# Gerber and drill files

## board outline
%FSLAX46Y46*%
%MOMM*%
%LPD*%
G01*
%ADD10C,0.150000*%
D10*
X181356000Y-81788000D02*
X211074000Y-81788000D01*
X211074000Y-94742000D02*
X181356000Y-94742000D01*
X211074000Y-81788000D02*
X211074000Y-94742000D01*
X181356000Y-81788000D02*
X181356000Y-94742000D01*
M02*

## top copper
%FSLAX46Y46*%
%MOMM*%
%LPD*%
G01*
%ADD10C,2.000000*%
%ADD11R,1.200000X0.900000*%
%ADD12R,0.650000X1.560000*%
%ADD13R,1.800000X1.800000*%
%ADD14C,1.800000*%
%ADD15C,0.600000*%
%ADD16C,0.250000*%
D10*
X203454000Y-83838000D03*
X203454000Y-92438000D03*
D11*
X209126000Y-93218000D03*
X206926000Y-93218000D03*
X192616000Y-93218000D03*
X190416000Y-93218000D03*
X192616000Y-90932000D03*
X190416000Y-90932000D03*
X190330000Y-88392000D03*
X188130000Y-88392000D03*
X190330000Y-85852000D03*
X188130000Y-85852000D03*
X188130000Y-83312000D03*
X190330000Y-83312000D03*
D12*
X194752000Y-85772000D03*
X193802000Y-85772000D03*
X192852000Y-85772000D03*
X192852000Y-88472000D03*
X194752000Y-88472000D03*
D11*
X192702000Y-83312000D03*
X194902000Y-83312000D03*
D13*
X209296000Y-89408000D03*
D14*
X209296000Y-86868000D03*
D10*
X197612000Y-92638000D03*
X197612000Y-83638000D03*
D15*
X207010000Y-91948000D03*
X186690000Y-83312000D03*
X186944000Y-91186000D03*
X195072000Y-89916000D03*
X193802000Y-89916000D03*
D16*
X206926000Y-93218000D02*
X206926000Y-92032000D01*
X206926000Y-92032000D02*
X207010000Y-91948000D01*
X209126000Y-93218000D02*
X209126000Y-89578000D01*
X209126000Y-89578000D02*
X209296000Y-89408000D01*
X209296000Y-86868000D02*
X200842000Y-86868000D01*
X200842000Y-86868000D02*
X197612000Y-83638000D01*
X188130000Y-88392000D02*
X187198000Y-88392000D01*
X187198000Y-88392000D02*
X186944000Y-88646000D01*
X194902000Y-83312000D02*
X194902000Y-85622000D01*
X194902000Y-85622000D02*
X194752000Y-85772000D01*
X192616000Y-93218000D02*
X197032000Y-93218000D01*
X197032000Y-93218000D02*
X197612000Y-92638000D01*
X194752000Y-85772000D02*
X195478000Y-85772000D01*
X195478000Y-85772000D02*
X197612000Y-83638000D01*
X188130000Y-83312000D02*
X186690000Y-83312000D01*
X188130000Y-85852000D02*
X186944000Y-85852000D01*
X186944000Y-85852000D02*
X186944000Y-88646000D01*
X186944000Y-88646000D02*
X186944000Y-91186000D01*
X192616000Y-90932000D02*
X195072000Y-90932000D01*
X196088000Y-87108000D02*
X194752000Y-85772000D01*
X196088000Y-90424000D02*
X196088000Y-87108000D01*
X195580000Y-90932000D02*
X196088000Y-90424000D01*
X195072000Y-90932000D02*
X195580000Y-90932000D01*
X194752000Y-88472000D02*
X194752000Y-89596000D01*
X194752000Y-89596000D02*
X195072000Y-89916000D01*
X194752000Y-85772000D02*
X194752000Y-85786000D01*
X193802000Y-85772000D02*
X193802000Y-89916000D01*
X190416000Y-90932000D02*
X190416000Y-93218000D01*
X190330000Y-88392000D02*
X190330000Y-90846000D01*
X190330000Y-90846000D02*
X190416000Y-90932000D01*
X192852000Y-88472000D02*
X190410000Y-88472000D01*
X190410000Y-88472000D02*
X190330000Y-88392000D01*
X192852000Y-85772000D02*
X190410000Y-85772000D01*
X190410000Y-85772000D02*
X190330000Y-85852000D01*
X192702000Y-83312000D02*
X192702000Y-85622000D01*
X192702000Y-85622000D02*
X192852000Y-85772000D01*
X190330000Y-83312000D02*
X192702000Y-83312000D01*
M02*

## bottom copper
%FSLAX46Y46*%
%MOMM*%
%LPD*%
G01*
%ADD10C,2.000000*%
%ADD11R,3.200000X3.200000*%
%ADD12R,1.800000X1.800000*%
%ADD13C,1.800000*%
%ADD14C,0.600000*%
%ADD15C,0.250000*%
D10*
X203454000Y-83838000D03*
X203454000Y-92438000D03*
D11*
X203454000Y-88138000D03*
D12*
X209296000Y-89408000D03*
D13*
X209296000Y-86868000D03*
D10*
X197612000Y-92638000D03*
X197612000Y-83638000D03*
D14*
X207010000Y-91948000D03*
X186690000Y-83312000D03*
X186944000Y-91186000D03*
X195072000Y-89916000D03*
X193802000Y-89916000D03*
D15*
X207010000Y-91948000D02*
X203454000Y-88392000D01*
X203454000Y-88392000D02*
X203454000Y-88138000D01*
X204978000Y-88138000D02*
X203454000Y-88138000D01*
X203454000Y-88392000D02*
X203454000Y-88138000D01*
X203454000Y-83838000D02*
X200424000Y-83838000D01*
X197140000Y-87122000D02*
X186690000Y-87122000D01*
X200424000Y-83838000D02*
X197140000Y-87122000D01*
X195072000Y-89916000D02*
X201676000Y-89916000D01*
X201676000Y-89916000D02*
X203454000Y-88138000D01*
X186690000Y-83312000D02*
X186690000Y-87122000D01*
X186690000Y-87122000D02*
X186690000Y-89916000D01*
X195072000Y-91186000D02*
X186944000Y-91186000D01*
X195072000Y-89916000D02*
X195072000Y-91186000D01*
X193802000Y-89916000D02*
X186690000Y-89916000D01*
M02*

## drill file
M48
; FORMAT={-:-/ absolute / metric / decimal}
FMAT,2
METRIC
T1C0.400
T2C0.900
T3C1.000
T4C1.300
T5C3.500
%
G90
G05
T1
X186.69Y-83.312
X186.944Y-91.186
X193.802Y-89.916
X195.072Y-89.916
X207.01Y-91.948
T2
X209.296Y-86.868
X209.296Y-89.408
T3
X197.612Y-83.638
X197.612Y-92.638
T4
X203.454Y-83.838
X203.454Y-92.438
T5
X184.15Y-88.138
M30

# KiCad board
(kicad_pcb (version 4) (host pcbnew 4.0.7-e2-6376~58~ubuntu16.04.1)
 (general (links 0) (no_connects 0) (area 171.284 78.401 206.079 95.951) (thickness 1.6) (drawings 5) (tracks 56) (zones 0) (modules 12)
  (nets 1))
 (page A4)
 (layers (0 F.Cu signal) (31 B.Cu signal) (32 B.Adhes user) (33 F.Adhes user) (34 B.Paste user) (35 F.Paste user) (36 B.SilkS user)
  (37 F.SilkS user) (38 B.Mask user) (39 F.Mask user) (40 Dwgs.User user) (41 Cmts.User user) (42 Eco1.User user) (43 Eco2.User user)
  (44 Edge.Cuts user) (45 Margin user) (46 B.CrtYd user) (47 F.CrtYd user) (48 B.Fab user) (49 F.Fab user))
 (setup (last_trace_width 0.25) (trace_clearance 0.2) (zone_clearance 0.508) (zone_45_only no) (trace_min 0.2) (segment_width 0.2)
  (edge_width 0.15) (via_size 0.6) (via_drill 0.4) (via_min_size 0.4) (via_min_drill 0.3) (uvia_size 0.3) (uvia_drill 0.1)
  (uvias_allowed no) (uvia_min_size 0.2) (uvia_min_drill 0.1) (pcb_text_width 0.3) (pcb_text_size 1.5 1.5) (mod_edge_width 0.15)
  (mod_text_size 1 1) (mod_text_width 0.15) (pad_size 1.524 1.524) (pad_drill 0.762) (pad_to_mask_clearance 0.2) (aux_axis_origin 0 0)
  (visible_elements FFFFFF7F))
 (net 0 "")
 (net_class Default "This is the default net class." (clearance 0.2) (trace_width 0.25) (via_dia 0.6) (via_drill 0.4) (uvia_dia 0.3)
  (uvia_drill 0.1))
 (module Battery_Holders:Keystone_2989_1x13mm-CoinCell (layer B.Cu) (at 203.454 88.138 270)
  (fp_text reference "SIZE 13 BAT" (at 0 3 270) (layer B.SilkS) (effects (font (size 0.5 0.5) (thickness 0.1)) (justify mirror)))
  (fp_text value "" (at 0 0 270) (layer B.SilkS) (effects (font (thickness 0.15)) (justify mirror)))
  (pad 1 thru_hole circle (at -4.3 0 270) (size 2 2) (drill 1.3) (layers *.Cu *.Mask))
  (pad 1 thru_hole circle (at 4.3 0 270) (size 2 2) (drill 1.3) (layers *.Cu *.Mask))
  (pad 2 smd rect (at 0 0 270) (size 3.2 3.2) (layers B.Cu B.Mask)))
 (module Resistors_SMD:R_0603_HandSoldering (layer F.Cu) (at 208.026 93.218 180)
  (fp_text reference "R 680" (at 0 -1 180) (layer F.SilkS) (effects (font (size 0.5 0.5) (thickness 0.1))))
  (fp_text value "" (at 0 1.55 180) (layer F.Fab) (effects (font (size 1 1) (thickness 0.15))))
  (pad 1 smd rect (at -1.1 0 180) (size 1.2 0.9) (layers F.Cu F.Paste F.Mask))
  (pad 2 smd rect (at 1.1 0 180) (size 1.2 0.9) (layers F.Cu F.Paste F.Mask)))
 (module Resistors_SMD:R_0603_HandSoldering (layer F.Cu) (at 191.516 93.218 180)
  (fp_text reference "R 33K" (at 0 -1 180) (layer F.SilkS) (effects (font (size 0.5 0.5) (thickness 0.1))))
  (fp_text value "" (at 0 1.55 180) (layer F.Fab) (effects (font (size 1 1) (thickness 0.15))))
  (pad 1 smd rect (at -1.1 0 180) (size 1.2 0.9) (layers F.Cu F.Paste F.Mask))
  (pad 2 smd rect (at 1.1 0 180) (size 1.2 0.9) (layers F.Cu F.Paste F.Mask)))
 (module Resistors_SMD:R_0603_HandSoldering (layer F.Cu) (at 191.516 90.932 180)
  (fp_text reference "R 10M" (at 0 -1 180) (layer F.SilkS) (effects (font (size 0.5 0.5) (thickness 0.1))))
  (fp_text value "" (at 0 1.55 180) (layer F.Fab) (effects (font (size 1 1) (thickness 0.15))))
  (pad 1 smd rect (at -1.1 0 180) (size 1.2 0.9) (layers F.Cu F.Paste F.Mask))
  (pad 2 smd rect (at 1.1 0 180) (size 1.2 0.9) (layers F.Cu F.Paste F.Mask)))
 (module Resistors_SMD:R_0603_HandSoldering (layer F.Cu) (at 189.23 88.392 180)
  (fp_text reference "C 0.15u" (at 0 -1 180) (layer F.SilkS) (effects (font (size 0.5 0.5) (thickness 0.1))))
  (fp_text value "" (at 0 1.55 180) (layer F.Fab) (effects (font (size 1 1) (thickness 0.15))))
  (pad 1 smd rect (at -1.1 0 180) (size 1.2 0.9) (layers F.Cu F.Paste F.Mask))
  (pad 2 smd rect (at 1.1 0 180) (size 1.2 0.9) (layers F.Cu F.Paste F.Mask)))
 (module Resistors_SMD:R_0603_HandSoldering (layer F.Cu) (at 189.23 85.852 180)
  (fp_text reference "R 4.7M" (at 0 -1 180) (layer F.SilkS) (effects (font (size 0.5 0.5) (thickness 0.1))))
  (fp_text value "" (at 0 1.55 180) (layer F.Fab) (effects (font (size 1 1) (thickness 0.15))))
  (pad 1 smd rect (at -1.1 0 180) (size 1.2 0.9) (layers F.Cu F.Paste F.Mask))
  (pad 2 smd rect (at 1.1 0 180) (size 1.2 0.9) (layers F.Cu F.Paste F.Mask)))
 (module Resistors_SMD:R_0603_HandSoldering (layer F.Cu) (at 189.23 83.312)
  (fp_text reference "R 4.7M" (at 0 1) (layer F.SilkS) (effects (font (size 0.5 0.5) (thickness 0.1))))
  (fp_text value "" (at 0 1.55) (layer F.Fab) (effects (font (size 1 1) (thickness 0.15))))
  (pad 1 smd rect (at -1.1 0) (size 1.2 0.9) (layers F.Cu F.Paste F.Mask))
  (pad 2 smd rect (at 1.1 0) (size 1.2 0.9) (layers F.Cu F.Paste F.Mask)))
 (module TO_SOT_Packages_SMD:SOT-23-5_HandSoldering (layer F.Cu) (at 193.802 87.122 270)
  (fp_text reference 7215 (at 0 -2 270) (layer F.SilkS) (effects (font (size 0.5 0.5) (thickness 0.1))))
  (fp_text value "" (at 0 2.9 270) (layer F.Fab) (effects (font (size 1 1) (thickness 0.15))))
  (pad 1 smd rect (at -1.35 -0.95 270) (size 1.56 0.65) (layers F.Cu F.Paste F.Mask))
  (pad 2 smd rect (at -1.35 0 270) (size 1.56 0.65) (layers F.Cu F.Paste F.Mask))
  (pad 3 smd rect (at -1.35 0.95 270) (size 1.56 0.65) (layers F.Cu F.Paste F.Mask))
  (pad 4 smd rect (at 1.35 0.95 270) (size 1.56 0.65) (layers F.Cu F.Paste F.Mask))
  (pad 5 smd rect (at 1.35 -0.95 270) (size 1.56 0.65) (layers F.Cu F.Paste F.Mask)))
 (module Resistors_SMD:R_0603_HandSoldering (layer F.Cu) (at 193.802 83.312)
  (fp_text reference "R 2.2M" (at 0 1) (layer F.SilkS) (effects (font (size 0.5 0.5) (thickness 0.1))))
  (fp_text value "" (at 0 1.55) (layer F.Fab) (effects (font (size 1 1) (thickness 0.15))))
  (pad 1 smd rect (at -1.1 0) (size 1.2 0.9) (layers F.Cu F.Paste F.Mask))
  (pad 2 smd rect (at 1.1 0) (size 1.2 0.9) (layers F.Cu F.Paste F.Mask)))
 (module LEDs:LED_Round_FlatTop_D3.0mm (layer F.Cu) (at 209.296 89.408 90)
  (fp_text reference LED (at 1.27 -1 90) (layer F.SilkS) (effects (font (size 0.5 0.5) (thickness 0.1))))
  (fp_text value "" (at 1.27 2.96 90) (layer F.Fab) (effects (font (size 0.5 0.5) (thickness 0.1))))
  (pad 1 thru_hole rect (at 0 0 90) (size 1.8 1.8) (drill 0.9) (layers *.Cu *.Mask))
  (pad 2 thru_hole circle (at 2.54 0 90) (size 1.8 1.8) (drill 0.9) (layers *.Cu *.Mask)))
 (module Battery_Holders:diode (layer F.Cu) (at 197.612 88.138 90)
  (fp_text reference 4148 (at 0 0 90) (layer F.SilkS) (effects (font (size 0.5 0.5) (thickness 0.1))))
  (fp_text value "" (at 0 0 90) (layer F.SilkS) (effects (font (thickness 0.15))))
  (pad 1 thru_hole circle (at -4.5 0 90) (size 2 2) (drill 1) (layers *.Cu *.Mask))
  (pad 2 thru_hole circle (at 4.5 0 90) (size 2 2) (drill 1) (layers *.Cu *.Mask)))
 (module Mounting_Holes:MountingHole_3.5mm (layer F.Cu) (at 184.15 88.138)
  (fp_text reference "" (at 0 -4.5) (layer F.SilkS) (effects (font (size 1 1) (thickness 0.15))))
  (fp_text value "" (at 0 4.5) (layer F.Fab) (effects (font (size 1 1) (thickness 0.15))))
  (pad 1 np_thru_hole circle (at 0 0) (size 3.5 3.5) (drill 3.5) (layers *.Cu *.Mask)))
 (gr_line (start 181.356 81.788) (end 211.074 81.788) (angle 90) (layer Edge.Cuts) (width 0.15))
 (gr_line (start 211.074 94.742) (end 181.356 94.742) (angle 90) (layer Edge.Cuts) (width 0.15))
 (gr_line (start 211.074 81.788) (end 211.074 94.742) (angle 90) (layer Edge.Cuts) (width 0.15))
 (gr_line (start 181.356 81.788) (end 181.356 94.742) (angle 90) (layer Edge.Cuts) (width 0.15))
 (segment (start 206.926 93.218) (end 206.926 92.032) (width 0.25) (layer F.Cu) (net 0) (status 400000))
 (segment (start 207.01 91.948) (end 203.454 88.392) (width 0.25) (layer B.Cu) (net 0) (status 800000))
 (via (at 207.01 91.948) (size 0.6) (drill 0.4) (layers F.Cu B.Cu) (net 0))
 (segment (start 206.926 92.032) (end 207.01 91.948) (width 0.25) (layer F.Cu) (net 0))
 (segment (start 203.454 88.392) (end 203.454 88.138) (width 0.25) (layer B.Cu) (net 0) (status C00000))
 (segment (start 209.126 93.218) (end 209.126 89.578) (width 0.25) (layer F.Cu) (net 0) (status C00000))
 (segment (start 209.126 89.578) (end 209.296 89.408) (width 0.25) (layer F.Cu) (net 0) (status C00000))
 (segment (start 209.296 86.868) (end 200.842 86.868) (width 0.25) (layer F.Cu) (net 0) (status 400000))
 (segment (start 200.842 86.868) (end 197.612 83.638) (width 0.25) (layer F.Cu) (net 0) (status 800000))
 (segment (start 204.978 88.138) (end 203.454 88.138) (width 0.25) (layer B.Cu) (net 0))
 (segment (start 188.13 88.392) (end 187.198 88.392) (width 0.25) (layer F.Cu) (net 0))
 (segment (start 187.198 88.392) (end 186.944 88.646) (width 0.25) (layer F.Cu) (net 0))
 (segment (start 203.454 88.392) (end 203.454 88.138) (width 0.25) (layer B.Cu) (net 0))
 (segment (start 194.902 83.312) (end 194.902 85.622) (width 0.25) (layer F.Cu) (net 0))
 (segment (start 194.902 85.622) (end 194.752 85.772) (width 0.25) (layer F.Cu) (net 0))
 (segment (start 203.454 83.838) (end 200.424 83.838) (width 0.25) (layer B.Cu) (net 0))
 (segment (start 197.14 87.122) (end 186.69 87.122) (width 0.25) (layer B.Cu) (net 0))
 (segment (start 200.424 83.838) (end 197.14 87.122) (width 0.25) (layer B.Cu) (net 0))
 (segment (start 195.072 89.916) (end 201.676 89.916) (width 0.25) (layer B.Cu) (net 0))
 (segment (start 201.676 89.916) (end 203.454 88.138) (width 0.25) (layer B.Cu) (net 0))
 (segment (start 192.616 93.218) (end 197.032 93.218) (width 0.25) (layer F.Cu) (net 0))
 (segment (start 197.032 93.218) (end 197.612 92.638) (width 0.25) (layer F.Cu) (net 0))
 (segment (start 194.752 85.772) (end 195.478 85.772) (width 0.25) (layer F.Cu) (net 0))
 (segment (start 195.478 85.772) (end 197.612 83.638) (width 0.25) (layer F.Cu) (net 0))
 (segment (start 188.13 83.312) (end 186.69 83.312) (width 0.25) (layer F.Cu) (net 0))
 (segment (start 186.69 83.312) (end 186.69 87.122) (width 0.25) (layer B.Cu) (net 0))
 (segment (start 186.69 87.122) (end 186.69 89.916) (width 0.25) (layer B.Cu) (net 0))
 (via (at 186.69 83.312) (size 0.6) (drill 0.4) (layers F.Cu B.Cu) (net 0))
 (segment (start 188.13 85.852) (end 186.944 85.852) (width 0.25) (layer F.Cu) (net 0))
 (via (at 186.944 91.186) (size 0.6) (drill 0.4) (layers F.Cu B.Cu) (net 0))
 (segment (start 186.944 85.852) (end 186.944 88.646) (width 0.25) (layer F.Cu) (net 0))
 (segment (start 186.944 88.646) (end 186.944 91.186) (width 0.25) (layer F.Cu) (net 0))
 (segment (start 192.616 90.932) (end 195.072 90.932) (width 0.25) (layer F.Cu) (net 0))
 (segment (start 196.088 87.108) (end 194.752 85.772) (width 0.25) (layer F.Cu) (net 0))
 (segment (start 196.088 90.424) (end 196.088 87.108) (width 0.25) (layer F.Cu) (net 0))
 (segment (start 195.58 90.932) (end 196.088 90.424) (width 0.25) (layer F.Cu) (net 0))
 (segment (start 195.072 90.932) (end 195.58 90.932) (width 0.25) (layer F.Cu) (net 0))
 (segment (start 194.752 88.472) (end 194.752 89.596) (width 0.25) (layer F.Cu) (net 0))
 (segment (start 195.072 91.186) (end 186.944 91.186) (width 0.25) (layer B.Cu) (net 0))
 (segment (start 195.072 89.916) (end 195.072 91.186) (width 0.25) (layer B.Cu) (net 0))
 (via (at 195.072 89.916) (size 0.6) (drill 0.4) (layers F.Cu B.Cu) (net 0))
 (segment (start 194.752 89.596) (end 195.072 89.916) (width 0.25) (layer F.Cu) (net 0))
 (segment (start 194.752 85.772) (end 194.752 85.786) (width 0.25) (layer F.Cu) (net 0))
 (segment (start 193.802 85.772) (end 193.802 89.916) (width 0.25) (layer F.Cu) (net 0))
 (segment (start 193.802 89.916) (end 186.69 89.916) (width 0.25) (layer B.Cu) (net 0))
 (via (at 193.802 89.916) (size 0.6) (drill 0.4) (layers F.Cu B.Cu) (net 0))
 (segment (start 190.416 90.932) (end 190.416 93.218) (width 0.25) (layer F.Cu) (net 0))
 (segment (start 190.33 88.392) (end 190.33 90.846) (width 0.25) (layer F.Cu) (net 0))
 (segment (start 190.33 90.846) (end 190.416 90.932) (width 0.25) (layer F.Cu) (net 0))
 (segment (start 192.852 88.472) (end 190.41 88.472) (width 0.25) (layer F.Cu) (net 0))
 (segment (start 190.41 88.472) (end 190.33 88.392) (width 0.25) (layer F.Cu) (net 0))
 (segment (start 192.852 85.772) (end 190.41 85.772) (width 0.25) (layer F.Cu) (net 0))
 (segment (start 190.41 85.772) (end 190.33 85.852) (width 0.25) (layer F.Cu) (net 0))
 (segment (start 192.702 83.312) (end 192.702 85.622) (width 0.25) (layer F.Cu) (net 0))
 (segment (start 192.702 85.622) (end 192.852 85.772) (width 0.25) (layer F.Cu) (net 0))
 (segment (start 190.33 83.312) (end 192.702 83.312) (width 0.25) (layer F.Cu) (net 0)))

